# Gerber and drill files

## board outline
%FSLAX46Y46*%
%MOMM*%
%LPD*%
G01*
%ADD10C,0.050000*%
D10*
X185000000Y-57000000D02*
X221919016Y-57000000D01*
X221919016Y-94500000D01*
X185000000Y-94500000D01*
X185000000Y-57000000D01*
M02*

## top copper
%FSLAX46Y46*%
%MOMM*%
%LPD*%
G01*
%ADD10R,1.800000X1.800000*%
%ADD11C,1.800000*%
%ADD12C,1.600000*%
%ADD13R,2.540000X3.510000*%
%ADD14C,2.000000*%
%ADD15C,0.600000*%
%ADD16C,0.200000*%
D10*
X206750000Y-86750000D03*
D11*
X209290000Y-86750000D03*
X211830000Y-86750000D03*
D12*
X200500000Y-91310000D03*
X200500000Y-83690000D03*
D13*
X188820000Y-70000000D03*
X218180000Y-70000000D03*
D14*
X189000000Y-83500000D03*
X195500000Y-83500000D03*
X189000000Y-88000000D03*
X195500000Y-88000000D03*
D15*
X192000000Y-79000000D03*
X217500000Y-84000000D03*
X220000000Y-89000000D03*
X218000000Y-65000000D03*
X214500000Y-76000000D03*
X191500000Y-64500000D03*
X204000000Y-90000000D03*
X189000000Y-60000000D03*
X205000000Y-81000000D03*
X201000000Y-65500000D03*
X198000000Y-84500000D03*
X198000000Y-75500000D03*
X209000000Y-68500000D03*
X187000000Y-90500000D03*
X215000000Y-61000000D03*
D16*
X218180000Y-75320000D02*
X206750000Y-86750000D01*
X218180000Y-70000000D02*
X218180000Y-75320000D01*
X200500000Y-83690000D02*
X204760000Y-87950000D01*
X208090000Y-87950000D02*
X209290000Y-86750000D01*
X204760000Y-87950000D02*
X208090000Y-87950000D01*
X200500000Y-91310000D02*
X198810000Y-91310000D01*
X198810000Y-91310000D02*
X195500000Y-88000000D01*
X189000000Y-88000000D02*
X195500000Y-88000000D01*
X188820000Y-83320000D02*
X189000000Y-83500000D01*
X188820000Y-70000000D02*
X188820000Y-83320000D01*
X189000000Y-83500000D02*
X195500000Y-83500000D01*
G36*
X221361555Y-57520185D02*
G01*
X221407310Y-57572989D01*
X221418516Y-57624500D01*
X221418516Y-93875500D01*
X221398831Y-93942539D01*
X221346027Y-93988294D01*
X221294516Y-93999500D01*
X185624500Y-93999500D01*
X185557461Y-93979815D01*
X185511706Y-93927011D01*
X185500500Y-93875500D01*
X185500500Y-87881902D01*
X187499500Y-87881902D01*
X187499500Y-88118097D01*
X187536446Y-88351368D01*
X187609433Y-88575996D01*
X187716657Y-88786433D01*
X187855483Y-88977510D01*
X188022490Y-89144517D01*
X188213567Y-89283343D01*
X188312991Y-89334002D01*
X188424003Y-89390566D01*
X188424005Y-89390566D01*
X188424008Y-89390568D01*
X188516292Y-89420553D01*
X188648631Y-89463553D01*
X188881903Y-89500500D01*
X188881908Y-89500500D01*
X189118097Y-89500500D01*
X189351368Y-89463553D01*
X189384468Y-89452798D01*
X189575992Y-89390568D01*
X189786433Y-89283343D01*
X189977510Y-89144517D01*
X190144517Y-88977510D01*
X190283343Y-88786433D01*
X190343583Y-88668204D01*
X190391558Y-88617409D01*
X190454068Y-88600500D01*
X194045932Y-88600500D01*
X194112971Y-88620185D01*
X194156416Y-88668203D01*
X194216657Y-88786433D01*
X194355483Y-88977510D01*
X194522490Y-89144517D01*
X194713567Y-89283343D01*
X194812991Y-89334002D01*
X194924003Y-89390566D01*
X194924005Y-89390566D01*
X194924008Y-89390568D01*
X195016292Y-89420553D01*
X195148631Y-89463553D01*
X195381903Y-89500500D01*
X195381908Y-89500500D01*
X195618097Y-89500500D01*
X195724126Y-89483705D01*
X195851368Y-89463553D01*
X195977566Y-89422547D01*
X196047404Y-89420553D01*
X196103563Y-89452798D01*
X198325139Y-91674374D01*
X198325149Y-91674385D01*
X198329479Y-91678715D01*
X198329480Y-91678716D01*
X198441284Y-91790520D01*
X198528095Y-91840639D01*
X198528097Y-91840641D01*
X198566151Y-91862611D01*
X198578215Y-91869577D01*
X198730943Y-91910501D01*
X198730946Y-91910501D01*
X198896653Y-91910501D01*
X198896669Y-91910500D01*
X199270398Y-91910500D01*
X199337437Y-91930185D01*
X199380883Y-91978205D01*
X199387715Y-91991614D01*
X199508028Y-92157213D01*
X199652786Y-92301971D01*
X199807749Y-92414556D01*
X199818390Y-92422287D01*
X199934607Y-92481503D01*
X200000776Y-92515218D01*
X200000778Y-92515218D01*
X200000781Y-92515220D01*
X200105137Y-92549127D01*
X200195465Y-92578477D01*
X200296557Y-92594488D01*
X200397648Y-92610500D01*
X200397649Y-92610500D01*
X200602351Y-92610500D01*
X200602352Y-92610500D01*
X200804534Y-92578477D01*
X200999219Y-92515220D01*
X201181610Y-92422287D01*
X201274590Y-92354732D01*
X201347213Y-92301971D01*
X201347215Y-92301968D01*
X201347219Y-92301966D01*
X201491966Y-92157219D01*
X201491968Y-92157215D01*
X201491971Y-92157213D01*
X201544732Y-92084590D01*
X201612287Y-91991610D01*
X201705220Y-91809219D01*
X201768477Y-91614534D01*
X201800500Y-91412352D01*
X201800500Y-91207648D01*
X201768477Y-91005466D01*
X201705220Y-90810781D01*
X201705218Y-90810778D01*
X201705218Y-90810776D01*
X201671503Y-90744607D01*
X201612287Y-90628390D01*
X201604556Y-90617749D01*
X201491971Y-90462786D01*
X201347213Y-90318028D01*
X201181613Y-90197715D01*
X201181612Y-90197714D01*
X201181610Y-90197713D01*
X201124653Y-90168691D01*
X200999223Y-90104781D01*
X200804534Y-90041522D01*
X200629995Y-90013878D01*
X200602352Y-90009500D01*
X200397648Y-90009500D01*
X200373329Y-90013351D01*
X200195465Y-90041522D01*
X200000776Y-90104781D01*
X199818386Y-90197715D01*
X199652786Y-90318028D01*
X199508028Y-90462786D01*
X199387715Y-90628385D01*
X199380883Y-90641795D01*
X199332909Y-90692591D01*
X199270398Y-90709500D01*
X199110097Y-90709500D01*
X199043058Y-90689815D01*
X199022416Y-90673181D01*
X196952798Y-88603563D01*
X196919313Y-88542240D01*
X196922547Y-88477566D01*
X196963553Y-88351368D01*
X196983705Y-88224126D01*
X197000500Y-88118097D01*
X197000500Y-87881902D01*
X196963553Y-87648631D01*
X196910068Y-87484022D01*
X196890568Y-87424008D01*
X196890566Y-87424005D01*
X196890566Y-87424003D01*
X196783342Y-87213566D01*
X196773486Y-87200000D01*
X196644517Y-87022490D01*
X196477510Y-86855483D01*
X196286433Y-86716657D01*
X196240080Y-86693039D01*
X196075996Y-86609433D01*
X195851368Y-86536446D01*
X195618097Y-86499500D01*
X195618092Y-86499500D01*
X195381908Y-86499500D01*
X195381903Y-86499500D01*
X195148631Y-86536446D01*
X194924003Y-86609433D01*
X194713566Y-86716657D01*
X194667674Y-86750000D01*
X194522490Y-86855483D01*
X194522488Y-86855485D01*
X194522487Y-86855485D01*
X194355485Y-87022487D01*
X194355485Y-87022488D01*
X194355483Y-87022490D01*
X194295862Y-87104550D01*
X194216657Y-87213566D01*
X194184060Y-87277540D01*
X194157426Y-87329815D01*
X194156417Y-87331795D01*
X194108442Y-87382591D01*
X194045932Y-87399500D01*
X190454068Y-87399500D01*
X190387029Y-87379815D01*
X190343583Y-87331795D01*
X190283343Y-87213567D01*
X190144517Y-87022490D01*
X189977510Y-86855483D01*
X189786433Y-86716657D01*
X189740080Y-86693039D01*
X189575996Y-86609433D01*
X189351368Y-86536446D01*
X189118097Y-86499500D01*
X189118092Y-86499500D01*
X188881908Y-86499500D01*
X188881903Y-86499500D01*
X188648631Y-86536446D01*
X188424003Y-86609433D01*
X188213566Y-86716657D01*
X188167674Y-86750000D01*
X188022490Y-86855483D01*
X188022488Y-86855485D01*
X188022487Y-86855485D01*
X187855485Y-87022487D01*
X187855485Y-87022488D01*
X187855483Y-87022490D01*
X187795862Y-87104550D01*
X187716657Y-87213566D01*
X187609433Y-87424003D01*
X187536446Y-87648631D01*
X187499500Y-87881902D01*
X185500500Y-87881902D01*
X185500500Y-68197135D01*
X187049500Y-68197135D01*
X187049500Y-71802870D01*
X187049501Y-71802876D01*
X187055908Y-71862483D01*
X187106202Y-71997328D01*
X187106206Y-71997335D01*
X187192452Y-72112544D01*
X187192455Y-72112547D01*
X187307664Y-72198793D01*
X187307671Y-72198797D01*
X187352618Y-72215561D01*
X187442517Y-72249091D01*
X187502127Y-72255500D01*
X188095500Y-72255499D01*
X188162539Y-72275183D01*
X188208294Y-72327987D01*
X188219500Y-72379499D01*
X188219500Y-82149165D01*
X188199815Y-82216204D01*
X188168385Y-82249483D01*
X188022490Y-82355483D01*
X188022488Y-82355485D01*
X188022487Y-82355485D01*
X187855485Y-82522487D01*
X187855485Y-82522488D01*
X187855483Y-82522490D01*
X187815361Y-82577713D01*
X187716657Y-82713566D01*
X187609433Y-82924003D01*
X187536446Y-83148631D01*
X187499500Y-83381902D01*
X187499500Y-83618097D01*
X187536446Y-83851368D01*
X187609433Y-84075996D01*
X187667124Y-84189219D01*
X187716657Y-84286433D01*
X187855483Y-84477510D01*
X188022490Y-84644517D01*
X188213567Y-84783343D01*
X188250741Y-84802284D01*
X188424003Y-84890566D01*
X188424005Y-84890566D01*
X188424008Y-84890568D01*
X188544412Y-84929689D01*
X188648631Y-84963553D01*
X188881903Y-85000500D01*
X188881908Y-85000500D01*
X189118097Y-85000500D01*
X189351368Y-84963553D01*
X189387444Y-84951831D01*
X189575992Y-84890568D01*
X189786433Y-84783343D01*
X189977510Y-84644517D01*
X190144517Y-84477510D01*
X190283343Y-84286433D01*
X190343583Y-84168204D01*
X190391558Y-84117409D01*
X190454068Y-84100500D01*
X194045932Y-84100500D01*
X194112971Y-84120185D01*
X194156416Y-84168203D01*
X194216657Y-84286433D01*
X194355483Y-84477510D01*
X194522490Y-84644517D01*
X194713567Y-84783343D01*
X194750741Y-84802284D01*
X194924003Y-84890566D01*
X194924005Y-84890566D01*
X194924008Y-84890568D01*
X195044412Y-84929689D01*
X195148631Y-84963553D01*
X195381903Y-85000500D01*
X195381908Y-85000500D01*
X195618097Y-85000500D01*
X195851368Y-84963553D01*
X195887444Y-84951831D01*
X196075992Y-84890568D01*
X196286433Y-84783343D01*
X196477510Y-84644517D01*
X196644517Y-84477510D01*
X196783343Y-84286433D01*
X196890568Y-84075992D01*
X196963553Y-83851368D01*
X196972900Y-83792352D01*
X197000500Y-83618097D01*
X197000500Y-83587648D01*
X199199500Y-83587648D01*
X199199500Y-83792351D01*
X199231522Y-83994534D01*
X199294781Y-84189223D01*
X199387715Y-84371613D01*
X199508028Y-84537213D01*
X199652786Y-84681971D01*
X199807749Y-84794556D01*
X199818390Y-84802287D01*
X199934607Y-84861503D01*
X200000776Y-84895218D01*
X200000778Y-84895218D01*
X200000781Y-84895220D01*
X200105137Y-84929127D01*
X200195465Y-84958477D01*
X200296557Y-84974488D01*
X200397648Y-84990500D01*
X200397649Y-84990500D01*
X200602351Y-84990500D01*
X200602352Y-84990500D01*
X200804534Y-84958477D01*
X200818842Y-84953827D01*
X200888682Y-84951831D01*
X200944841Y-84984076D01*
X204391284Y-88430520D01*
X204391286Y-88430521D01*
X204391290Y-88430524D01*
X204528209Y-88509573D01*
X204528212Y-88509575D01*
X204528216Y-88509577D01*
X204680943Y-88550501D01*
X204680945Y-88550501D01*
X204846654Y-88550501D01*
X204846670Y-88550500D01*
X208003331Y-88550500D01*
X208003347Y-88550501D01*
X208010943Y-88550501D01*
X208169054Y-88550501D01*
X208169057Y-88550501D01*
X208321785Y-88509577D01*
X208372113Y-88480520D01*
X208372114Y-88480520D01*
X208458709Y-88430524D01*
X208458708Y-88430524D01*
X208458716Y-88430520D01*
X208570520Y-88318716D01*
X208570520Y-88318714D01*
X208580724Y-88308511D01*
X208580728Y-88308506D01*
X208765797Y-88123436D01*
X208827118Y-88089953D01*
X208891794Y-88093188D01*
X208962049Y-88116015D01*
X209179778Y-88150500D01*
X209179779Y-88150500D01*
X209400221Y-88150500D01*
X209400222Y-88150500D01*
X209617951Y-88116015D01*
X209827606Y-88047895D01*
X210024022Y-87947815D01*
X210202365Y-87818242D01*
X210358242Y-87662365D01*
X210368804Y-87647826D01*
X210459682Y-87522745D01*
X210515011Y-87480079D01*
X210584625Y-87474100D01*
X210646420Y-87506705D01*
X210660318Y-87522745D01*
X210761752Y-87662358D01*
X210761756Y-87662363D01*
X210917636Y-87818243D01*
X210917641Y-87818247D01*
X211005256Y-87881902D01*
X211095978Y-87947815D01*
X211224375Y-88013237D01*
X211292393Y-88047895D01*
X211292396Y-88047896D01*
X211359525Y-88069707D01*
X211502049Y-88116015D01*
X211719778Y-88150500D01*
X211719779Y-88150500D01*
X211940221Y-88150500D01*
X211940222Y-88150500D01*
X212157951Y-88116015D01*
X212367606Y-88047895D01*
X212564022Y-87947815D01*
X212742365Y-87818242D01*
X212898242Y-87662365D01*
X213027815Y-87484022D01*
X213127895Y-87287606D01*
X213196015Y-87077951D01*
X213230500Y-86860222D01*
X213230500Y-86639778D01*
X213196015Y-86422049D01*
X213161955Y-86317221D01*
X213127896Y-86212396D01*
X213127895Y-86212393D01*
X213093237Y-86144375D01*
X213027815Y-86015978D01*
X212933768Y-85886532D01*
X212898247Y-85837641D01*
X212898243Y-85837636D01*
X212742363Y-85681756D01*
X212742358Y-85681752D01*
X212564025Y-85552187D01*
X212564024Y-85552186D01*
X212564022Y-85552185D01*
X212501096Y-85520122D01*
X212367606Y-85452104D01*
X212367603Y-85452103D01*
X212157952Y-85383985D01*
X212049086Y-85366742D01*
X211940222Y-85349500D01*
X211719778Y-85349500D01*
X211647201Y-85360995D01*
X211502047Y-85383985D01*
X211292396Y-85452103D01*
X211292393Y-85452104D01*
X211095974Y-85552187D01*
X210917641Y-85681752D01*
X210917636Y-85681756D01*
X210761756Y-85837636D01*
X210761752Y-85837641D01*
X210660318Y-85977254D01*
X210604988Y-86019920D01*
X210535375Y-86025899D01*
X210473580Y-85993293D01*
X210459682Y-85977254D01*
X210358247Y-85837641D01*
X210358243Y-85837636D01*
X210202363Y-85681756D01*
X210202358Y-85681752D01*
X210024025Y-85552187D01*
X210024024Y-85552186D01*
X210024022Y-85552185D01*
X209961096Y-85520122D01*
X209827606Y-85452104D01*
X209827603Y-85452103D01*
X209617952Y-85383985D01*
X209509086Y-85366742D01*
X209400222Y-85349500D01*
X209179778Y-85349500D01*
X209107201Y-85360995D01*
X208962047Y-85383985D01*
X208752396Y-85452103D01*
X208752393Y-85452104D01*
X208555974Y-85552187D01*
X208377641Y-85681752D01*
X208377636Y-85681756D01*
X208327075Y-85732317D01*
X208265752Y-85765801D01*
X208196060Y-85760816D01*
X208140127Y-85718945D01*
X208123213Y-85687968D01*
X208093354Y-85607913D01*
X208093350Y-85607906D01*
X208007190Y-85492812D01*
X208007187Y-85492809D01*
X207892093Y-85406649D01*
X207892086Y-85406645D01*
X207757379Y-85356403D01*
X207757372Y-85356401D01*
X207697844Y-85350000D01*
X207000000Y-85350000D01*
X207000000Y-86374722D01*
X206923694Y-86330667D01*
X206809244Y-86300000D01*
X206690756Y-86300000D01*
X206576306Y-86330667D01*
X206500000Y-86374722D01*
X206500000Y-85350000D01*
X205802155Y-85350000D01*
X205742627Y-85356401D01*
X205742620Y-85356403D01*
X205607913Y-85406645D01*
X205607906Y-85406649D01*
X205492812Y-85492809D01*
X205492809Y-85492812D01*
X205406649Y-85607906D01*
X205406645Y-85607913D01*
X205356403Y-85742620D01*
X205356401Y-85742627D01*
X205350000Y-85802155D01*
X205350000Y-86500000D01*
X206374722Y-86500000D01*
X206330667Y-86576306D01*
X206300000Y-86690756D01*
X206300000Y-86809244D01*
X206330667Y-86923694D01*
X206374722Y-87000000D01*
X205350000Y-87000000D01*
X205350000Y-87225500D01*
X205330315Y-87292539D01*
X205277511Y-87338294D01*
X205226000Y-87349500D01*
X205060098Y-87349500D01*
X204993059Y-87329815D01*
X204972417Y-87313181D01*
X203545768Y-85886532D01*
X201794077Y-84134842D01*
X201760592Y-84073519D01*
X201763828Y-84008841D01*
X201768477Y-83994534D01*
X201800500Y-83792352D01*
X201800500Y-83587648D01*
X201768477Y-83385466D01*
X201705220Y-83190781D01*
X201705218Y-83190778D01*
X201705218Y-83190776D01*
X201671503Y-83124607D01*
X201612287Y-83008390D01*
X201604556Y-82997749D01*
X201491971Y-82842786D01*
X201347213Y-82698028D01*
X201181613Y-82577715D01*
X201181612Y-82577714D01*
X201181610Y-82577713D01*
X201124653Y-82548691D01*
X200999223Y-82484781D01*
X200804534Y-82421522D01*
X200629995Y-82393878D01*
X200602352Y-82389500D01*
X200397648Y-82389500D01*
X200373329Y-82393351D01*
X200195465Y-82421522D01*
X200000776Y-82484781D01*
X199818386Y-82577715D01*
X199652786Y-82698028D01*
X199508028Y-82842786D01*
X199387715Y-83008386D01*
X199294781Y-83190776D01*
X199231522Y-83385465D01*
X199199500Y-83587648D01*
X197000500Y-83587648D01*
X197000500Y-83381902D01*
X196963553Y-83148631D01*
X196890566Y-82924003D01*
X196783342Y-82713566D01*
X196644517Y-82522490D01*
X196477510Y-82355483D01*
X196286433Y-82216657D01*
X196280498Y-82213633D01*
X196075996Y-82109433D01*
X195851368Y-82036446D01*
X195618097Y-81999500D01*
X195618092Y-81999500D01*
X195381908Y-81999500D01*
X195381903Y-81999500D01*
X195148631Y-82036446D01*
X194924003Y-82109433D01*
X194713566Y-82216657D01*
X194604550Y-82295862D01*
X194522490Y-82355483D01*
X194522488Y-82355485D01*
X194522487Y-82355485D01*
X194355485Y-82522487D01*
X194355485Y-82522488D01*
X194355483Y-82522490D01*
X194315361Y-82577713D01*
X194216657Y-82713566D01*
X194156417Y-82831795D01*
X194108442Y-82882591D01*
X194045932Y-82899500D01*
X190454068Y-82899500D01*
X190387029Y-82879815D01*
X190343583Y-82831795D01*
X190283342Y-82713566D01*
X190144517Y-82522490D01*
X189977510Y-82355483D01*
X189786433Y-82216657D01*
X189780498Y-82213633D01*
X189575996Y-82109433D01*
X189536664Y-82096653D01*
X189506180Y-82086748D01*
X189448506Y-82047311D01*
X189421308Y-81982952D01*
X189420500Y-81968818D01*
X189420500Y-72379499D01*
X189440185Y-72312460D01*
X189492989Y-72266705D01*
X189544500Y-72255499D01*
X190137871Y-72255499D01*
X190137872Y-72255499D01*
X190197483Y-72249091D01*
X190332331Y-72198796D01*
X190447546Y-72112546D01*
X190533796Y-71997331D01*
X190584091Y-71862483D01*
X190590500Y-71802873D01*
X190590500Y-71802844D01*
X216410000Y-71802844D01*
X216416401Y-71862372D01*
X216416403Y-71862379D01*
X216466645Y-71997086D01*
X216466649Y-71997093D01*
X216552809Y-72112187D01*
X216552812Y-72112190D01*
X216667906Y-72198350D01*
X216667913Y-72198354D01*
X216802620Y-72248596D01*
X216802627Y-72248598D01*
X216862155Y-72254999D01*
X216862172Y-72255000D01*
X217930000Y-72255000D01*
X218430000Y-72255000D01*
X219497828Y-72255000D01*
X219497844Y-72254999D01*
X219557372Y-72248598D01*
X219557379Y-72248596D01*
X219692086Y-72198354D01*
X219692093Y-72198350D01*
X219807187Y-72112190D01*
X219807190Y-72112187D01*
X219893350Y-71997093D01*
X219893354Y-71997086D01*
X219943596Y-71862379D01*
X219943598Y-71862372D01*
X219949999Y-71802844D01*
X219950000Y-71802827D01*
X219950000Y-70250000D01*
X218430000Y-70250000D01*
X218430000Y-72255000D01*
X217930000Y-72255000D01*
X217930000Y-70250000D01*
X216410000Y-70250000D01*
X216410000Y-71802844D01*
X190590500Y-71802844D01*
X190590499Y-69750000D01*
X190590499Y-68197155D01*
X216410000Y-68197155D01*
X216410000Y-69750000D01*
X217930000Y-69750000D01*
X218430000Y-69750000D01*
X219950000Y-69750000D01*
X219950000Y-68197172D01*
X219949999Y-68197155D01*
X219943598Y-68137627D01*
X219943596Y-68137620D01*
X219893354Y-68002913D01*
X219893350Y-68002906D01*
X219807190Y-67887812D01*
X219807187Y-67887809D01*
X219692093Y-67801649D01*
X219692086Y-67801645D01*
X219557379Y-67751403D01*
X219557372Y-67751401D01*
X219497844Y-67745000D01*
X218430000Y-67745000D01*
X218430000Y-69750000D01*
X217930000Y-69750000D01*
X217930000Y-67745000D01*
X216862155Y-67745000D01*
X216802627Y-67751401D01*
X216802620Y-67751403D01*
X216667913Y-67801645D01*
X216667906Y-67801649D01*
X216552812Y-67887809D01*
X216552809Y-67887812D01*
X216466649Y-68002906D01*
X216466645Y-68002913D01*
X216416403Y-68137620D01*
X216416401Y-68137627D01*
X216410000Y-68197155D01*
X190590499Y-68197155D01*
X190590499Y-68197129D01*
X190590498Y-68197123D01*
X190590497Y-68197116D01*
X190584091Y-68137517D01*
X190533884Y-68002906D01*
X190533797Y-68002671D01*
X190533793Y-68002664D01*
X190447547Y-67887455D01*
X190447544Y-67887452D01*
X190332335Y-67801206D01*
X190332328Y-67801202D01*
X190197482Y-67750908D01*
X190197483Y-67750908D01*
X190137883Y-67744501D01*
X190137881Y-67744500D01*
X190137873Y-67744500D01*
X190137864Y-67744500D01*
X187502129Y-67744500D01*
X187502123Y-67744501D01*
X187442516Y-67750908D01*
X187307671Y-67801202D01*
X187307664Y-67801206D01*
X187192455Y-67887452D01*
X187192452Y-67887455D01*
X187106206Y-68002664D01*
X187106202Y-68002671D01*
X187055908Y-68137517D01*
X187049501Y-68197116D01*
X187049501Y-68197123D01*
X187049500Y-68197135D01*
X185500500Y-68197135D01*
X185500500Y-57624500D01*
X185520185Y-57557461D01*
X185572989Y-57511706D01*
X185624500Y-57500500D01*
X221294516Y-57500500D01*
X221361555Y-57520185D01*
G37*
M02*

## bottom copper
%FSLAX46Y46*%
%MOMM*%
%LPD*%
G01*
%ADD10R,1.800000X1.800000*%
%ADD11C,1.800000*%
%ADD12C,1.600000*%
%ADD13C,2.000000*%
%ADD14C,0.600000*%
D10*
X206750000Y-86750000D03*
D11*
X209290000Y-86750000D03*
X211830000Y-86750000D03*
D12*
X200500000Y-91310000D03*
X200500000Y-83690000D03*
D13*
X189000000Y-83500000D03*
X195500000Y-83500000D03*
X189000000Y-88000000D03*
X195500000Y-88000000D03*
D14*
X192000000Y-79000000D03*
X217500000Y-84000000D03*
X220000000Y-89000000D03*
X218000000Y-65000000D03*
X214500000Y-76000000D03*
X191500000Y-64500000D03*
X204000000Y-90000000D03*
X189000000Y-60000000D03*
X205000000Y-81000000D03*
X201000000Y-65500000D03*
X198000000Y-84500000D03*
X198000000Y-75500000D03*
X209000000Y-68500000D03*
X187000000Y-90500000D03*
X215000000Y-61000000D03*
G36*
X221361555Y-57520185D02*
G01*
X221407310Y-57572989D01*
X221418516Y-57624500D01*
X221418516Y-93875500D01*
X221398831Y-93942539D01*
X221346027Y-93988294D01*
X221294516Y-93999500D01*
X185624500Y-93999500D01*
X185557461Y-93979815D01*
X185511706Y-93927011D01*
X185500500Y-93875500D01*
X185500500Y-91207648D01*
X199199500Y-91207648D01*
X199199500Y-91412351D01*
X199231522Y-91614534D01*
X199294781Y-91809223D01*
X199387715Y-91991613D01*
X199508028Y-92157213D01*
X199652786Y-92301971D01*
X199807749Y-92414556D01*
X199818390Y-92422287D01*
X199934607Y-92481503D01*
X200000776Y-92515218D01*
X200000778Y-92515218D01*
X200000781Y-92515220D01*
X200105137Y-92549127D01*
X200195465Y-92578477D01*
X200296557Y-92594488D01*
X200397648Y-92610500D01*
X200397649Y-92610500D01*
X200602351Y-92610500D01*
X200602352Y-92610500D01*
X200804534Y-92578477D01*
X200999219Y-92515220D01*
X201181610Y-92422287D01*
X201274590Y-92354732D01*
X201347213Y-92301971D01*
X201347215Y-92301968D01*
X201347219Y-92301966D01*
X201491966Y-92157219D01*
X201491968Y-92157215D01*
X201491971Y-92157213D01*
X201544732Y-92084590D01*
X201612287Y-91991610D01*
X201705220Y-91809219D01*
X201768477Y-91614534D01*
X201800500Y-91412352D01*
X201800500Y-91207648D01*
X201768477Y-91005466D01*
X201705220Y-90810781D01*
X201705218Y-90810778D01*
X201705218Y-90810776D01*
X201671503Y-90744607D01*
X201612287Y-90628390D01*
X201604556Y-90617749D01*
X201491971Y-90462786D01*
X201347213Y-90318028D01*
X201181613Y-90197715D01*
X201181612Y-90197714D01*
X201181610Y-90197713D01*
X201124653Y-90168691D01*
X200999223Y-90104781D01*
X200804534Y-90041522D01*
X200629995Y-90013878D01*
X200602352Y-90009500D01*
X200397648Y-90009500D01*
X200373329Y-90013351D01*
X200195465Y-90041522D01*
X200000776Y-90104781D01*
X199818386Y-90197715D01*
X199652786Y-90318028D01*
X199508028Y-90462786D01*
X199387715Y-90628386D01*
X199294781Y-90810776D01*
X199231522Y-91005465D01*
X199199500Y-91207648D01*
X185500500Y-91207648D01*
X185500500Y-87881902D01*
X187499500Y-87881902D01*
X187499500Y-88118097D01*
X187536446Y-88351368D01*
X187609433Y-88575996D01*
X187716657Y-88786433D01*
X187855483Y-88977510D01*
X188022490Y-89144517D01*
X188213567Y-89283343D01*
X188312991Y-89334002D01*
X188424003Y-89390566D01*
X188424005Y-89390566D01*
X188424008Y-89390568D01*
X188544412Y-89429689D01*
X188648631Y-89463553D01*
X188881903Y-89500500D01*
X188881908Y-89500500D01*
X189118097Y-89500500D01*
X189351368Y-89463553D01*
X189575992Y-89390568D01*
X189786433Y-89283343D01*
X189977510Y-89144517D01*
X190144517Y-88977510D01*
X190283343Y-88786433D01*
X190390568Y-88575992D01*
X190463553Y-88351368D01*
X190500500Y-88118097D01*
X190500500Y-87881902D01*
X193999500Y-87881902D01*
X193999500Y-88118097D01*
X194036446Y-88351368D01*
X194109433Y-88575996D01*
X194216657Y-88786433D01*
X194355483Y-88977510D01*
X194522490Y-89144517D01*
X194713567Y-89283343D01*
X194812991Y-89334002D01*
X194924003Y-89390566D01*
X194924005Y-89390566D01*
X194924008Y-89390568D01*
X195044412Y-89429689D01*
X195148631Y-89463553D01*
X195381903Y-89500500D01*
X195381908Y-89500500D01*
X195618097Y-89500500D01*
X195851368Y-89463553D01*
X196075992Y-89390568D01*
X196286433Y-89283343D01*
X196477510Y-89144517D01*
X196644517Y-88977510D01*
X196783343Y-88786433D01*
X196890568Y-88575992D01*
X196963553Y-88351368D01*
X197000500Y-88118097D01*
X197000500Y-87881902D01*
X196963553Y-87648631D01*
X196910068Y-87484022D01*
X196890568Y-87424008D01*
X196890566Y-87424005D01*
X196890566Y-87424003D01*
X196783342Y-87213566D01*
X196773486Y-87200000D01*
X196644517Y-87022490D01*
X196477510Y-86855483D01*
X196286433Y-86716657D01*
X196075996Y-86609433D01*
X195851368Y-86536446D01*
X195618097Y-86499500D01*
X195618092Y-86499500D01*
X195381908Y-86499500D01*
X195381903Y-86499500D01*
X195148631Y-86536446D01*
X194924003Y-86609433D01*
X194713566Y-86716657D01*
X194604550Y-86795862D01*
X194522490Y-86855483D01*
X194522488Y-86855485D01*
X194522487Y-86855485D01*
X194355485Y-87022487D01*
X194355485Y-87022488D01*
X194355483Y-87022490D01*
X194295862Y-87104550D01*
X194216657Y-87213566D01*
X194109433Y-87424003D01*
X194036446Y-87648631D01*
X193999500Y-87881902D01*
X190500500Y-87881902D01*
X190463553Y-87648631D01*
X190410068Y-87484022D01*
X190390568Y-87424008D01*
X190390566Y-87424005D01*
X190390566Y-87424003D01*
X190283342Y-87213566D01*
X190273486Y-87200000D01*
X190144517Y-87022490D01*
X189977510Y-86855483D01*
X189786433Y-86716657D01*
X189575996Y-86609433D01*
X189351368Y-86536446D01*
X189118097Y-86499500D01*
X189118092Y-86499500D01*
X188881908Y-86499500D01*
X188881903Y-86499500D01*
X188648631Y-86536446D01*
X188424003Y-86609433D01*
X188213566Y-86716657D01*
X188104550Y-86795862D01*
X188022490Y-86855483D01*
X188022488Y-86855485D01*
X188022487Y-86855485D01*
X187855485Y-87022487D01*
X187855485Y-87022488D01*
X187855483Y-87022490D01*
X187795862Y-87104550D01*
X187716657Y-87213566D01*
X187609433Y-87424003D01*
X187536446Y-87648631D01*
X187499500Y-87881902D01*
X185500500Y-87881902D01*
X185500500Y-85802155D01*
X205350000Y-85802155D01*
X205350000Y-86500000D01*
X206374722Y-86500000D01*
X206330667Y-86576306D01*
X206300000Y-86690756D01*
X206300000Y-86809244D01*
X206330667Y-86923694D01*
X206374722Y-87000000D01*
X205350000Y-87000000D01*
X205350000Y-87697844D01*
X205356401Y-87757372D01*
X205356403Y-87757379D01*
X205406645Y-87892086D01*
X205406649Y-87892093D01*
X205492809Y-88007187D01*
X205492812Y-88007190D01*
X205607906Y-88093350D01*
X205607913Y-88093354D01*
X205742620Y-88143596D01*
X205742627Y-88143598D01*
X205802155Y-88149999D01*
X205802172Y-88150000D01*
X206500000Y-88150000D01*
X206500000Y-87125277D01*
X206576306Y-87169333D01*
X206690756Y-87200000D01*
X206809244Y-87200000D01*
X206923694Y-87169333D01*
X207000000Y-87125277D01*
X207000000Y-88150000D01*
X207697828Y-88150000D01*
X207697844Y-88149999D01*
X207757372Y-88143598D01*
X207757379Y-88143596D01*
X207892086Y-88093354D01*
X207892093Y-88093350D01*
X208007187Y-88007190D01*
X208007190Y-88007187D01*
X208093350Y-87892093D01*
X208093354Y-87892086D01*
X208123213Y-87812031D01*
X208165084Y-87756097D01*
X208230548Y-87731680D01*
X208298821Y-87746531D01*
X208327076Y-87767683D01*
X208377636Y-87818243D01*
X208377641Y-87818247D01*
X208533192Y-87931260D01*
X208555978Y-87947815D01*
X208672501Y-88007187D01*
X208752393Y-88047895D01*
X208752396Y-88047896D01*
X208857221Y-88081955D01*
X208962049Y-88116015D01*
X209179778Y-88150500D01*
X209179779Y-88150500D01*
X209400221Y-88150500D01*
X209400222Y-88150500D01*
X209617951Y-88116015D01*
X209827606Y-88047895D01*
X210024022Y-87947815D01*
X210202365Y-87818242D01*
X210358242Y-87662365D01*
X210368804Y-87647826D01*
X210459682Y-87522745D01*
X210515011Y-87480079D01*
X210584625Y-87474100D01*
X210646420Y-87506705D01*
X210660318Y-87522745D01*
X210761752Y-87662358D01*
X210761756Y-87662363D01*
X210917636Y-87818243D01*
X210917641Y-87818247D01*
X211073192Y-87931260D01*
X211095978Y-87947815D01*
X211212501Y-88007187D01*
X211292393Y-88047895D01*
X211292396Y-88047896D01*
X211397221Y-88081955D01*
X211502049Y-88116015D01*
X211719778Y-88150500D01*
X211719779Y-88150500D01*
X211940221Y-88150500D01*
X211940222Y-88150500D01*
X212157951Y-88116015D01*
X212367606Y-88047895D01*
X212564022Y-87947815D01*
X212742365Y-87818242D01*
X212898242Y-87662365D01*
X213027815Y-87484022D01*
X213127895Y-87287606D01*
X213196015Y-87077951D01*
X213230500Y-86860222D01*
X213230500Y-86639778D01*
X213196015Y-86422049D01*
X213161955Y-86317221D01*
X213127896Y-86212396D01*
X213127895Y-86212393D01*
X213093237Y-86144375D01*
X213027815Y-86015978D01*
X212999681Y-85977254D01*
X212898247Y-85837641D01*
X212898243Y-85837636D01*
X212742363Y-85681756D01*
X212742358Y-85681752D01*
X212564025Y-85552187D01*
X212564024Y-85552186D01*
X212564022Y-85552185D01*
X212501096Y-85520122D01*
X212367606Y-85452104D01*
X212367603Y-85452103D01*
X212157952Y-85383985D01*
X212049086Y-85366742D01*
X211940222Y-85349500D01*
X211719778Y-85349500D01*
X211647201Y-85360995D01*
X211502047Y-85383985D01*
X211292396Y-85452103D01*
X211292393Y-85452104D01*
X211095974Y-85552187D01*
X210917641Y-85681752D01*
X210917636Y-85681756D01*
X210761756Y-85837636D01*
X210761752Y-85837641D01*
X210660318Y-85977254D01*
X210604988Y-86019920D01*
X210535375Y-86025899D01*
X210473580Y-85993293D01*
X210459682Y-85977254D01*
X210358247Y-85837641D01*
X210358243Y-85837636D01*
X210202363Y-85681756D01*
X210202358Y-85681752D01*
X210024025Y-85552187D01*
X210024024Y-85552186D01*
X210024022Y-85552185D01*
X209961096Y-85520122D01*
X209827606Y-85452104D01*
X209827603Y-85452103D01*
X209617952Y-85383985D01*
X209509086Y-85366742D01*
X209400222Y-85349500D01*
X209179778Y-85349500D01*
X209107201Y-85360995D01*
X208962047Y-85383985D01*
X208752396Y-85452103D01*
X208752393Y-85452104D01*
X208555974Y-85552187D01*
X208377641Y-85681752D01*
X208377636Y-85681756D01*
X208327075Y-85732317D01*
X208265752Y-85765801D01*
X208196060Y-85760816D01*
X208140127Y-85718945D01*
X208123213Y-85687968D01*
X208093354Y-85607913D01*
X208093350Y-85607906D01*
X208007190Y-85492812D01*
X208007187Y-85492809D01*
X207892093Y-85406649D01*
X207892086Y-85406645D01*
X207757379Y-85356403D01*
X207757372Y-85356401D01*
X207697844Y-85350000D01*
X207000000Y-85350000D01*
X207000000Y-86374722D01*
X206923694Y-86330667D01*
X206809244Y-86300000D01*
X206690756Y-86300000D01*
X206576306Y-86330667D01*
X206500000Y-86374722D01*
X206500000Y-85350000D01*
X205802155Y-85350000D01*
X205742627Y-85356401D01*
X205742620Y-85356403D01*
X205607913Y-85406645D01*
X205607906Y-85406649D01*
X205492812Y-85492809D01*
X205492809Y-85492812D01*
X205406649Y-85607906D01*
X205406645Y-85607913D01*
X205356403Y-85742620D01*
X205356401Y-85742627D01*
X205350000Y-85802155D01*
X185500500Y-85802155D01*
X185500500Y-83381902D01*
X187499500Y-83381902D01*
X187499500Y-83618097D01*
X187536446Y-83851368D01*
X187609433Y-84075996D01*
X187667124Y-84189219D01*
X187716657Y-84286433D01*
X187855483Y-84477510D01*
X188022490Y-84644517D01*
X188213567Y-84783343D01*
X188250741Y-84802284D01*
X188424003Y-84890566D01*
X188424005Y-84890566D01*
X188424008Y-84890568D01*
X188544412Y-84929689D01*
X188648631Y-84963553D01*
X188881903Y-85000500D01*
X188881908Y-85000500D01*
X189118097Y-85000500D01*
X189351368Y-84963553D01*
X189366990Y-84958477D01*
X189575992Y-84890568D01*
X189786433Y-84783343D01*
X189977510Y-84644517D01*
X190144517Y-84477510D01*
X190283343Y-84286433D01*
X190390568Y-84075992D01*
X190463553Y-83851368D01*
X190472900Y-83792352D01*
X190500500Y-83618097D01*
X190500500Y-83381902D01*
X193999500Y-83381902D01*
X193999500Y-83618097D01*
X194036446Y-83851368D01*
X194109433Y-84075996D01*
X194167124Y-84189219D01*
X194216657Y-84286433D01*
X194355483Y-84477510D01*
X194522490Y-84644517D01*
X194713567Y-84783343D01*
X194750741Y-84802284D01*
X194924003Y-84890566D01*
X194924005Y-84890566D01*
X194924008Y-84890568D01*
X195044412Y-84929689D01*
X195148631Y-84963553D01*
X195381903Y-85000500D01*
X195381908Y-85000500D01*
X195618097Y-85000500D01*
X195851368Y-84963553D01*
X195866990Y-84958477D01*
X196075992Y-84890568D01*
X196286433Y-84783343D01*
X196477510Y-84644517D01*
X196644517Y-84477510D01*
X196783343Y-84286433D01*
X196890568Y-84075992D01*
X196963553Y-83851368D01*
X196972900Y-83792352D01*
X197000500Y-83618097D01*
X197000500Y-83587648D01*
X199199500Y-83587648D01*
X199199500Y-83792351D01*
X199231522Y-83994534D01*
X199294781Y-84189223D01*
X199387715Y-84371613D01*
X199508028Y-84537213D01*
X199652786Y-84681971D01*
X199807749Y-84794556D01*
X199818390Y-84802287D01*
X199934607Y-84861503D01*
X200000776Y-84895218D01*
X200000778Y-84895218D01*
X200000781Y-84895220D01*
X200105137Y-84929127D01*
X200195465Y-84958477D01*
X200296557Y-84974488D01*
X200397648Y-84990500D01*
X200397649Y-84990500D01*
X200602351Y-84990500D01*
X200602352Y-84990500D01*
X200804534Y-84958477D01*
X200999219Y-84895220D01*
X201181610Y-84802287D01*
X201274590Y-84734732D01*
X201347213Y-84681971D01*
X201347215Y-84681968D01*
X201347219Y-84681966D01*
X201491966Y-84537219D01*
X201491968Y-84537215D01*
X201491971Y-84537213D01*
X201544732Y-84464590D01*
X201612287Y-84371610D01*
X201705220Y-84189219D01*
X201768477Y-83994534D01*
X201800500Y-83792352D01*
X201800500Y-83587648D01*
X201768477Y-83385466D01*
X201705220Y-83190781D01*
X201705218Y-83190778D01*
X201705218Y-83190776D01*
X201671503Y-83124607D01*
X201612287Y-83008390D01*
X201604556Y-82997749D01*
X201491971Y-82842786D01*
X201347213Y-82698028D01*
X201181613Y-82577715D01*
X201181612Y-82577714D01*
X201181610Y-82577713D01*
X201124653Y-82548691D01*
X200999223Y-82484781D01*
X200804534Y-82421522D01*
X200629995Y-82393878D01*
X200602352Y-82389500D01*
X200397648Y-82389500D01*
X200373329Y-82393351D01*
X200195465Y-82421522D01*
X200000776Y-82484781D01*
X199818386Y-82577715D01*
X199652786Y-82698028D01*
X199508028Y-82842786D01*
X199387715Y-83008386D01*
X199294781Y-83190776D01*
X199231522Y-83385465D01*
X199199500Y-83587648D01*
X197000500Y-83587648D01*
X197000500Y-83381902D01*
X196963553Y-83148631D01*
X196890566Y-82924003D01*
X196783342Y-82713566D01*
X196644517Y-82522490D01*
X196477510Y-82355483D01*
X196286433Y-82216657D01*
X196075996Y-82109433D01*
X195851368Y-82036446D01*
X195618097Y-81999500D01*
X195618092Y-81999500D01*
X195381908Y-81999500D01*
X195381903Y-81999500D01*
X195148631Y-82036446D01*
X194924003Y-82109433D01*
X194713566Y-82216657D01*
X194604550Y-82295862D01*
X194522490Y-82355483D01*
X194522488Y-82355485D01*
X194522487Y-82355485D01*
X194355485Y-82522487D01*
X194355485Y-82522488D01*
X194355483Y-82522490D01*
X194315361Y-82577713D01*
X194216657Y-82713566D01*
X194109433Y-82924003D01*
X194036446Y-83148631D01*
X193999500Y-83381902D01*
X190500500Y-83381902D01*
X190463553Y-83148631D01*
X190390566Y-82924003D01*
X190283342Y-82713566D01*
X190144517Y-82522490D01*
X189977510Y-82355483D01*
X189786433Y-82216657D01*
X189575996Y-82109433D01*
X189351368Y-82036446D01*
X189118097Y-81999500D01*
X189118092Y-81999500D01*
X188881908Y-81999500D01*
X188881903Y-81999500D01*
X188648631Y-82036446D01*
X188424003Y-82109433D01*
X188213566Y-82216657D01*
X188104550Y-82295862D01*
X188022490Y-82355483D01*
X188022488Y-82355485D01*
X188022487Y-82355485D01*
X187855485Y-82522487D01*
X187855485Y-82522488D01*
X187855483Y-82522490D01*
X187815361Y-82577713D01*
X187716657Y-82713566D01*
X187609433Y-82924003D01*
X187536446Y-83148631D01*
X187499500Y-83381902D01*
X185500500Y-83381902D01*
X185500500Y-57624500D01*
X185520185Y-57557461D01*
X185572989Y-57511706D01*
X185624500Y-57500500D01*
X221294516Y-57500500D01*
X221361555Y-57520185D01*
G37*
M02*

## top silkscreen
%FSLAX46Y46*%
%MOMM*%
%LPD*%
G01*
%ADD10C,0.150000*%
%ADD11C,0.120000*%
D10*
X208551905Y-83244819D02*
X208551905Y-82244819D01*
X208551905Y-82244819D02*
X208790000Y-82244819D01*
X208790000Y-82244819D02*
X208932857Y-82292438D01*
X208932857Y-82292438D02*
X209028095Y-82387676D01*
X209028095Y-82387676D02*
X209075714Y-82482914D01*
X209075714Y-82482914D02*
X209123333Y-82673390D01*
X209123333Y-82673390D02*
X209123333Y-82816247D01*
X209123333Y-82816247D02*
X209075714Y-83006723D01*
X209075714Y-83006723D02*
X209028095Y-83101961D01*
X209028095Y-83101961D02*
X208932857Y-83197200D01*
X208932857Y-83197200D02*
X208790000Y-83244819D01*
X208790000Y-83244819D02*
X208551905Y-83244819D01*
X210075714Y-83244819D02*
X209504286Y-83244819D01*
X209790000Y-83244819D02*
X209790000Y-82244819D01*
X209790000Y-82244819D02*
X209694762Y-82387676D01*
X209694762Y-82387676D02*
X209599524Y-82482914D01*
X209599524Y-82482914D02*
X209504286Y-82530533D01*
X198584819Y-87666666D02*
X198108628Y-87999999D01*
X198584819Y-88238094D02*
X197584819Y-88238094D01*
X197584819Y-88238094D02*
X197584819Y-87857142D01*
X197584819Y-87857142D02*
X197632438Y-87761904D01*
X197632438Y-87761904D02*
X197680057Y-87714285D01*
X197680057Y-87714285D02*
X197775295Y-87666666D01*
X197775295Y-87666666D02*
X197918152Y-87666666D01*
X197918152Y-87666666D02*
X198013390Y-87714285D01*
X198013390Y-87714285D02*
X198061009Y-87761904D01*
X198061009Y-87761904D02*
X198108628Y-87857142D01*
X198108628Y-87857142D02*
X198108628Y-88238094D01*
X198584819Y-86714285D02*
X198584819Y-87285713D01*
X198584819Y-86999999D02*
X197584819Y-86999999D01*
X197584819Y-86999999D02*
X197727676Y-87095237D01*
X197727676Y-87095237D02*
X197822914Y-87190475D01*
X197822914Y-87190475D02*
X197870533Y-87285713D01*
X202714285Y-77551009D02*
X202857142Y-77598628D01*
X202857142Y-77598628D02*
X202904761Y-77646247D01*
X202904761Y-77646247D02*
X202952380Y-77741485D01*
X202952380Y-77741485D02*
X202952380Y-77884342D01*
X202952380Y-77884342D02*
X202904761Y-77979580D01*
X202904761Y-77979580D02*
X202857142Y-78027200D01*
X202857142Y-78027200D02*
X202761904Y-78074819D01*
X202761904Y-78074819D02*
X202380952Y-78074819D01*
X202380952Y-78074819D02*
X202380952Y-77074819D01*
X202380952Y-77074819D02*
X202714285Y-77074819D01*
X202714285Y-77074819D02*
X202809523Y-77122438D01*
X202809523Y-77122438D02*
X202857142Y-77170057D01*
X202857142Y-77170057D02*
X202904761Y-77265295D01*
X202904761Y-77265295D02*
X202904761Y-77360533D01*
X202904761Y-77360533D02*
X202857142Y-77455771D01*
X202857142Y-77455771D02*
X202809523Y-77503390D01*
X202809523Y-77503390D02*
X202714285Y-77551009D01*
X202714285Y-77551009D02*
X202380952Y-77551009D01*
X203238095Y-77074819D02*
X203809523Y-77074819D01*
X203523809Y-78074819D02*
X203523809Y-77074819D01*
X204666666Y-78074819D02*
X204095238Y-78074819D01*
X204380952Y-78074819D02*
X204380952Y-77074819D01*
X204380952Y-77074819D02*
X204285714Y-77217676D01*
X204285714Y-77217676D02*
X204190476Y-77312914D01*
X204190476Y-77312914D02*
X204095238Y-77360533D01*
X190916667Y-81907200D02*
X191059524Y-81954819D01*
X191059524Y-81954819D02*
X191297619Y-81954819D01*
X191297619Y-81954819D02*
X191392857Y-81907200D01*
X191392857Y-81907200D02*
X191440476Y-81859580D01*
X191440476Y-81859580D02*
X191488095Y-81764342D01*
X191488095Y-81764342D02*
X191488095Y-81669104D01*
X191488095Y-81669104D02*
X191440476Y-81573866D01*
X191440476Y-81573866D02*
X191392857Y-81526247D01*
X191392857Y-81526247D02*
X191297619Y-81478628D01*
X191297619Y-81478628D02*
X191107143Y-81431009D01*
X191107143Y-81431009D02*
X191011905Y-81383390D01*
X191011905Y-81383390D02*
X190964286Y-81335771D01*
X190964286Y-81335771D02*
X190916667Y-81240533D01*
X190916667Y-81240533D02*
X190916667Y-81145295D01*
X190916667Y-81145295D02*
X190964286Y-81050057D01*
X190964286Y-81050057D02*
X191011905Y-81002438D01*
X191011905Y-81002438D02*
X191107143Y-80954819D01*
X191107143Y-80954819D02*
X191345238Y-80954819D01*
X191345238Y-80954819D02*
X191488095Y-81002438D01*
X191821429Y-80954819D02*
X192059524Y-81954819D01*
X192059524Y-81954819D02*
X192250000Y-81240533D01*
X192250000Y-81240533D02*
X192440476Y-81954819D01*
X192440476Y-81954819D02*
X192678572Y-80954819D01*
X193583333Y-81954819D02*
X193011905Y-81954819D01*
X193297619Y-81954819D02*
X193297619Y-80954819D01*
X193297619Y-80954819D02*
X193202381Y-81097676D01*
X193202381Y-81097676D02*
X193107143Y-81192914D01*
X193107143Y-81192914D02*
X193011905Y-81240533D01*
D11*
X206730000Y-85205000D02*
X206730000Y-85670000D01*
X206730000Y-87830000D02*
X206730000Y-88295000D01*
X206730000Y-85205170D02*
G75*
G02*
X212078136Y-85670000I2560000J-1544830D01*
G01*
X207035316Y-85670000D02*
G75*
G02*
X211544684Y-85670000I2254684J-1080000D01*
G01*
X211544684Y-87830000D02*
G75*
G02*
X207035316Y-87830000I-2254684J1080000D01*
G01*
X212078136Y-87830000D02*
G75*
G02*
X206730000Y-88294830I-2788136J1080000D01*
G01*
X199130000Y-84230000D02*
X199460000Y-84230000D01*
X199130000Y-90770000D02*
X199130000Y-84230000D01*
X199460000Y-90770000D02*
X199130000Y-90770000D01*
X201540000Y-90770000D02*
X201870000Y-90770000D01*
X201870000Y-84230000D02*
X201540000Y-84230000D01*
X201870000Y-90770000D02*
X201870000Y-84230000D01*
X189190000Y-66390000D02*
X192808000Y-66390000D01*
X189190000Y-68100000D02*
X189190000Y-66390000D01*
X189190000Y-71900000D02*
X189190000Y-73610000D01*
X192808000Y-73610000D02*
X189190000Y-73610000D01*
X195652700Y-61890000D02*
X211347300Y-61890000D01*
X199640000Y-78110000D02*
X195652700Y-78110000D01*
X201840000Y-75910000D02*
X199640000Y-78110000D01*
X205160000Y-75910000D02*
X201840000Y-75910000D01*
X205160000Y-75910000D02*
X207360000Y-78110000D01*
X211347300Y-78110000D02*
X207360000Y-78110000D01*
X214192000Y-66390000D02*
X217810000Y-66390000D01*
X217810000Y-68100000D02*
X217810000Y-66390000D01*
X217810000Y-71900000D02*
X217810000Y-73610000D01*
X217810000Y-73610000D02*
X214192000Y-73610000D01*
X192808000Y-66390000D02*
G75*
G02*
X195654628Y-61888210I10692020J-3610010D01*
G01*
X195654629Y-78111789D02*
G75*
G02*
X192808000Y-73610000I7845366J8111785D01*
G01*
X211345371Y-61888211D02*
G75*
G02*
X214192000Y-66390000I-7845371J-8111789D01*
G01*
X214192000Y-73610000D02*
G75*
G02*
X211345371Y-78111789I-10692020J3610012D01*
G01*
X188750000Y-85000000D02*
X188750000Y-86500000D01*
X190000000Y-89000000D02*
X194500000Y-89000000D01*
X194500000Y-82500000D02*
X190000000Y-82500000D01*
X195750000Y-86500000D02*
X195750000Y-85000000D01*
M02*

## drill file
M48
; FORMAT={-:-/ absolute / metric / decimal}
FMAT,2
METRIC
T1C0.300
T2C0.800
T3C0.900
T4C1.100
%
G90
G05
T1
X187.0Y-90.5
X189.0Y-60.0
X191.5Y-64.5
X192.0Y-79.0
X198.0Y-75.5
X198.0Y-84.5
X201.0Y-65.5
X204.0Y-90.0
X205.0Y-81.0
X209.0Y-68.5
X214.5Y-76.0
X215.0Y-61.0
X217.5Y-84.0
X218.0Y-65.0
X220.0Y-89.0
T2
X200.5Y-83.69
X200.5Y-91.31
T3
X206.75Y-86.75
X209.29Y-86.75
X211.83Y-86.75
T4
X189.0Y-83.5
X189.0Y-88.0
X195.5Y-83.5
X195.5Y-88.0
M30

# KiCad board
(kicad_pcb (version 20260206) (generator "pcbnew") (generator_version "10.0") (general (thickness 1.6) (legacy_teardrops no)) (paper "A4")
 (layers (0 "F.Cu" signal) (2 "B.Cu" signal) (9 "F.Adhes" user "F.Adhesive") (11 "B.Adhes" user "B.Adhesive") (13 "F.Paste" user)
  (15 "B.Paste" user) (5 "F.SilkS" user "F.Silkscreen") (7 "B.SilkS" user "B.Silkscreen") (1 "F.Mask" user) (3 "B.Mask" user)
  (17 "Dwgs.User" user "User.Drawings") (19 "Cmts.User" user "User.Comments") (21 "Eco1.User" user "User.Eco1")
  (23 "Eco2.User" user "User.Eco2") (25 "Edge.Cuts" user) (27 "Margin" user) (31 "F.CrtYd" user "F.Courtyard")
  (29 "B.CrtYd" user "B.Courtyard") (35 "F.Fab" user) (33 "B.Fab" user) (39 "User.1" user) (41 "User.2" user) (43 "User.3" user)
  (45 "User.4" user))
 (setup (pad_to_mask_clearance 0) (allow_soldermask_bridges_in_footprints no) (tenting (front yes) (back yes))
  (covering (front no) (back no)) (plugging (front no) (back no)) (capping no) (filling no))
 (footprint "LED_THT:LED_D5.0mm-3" (layer "F.Cu") (at 206.75 86.75)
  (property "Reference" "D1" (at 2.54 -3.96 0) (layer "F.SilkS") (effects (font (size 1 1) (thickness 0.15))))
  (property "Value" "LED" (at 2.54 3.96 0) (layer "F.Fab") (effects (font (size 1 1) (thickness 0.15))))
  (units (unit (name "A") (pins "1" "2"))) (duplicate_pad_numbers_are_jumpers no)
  (fp_line (start -0.02 -1.545) (end -0.02 -1.08) (stroke (width 0.12) (type solid)) (layer "F.SilkS"))
  (fp_line (start -0.02 1.08) (end -0.02 1.545) (stroke (width 0.12) (type solid)) (layer "F.SilkS"))
  (fp_arc (start -0.02 -1.54483) (mid 2.798898 -2.97877) (end 5.328136 -1.08) (stroke (width 0.12) (type solid)) (layer "F.SilkS"))
  (fp_arc (start 0.285316 -1.08) (mid 2.54 -2.5) (end 4.794684 -1.08) (stroke (width 0.12) (type solid)) (layer "F.SilkS"))
  (fp_arc (start 4.794684 1.08) (mid 2.54 2.5) (end 0.285316 1.08) (stroke (width 0.12) (type solid)) (layer "F.SilkS"))
  (fp_arc (start 5.328136 1.08) (mid 2.798898 2.97877) (end -0.02 1.54483) (stroke (width 0.12) (type solid)) (layer "F.SilkS"))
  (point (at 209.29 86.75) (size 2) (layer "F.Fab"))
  (pad "1" thru_hole rect (at 0 0) (size 1.8 1.8) (drill 0.9) (layers "*.Cu" "*.Mask") (remove_unused_layers no) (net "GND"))
  (pad "2" thru_hole circle (at 2.54 0) (size 1.8 1.8) (drill 0.9) (layers "*.Cu" "*.Mask") (remove_unused_layers no) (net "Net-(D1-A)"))
  (pad "3" thru_hole circle (at 5.08 0) (size 1.8 1.8) (drill 0.9) (layers "*.Cu" "*.Mask") (remove_unused_layers no)))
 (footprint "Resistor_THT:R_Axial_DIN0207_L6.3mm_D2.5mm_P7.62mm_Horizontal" (layer "F.Cu") (at 200.5 91.31 90)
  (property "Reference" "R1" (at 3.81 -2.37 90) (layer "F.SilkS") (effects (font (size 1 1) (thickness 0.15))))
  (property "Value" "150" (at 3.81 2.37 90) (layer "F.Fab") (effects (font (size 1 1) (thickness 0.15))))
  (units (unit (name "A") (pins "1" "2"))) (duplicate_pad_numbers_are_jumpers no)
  (fp_line (start 7.08 -1.37) (end 7.08 -1.04) (stroke (width 0.12) (type solid)) (layer "F.SilkS"))
  (fp_line (start 0.54 -1.37) (end 7.08 -1.37) (stroke (width 0.12) (type solid)) (layer "F.SilkS"))
  (fp_line (start 0.54 -1.04) (end 0.54 -1.37) (stroke (width 0.12) (type solid)) (layer "F.SilkS"))
  (fp_line (start 0.54 1.04) (end 0.54 1.37) (stroke (width 0.12) (type solid)) (layer "F.SilkS"))
  (fp_line (start 7.08 1.37) (end 7.08 1.04) (stroke (width 0.12) (type solid)) (layer "F.SilkS"))
  (fp_line (start 0.54 1.37) (end 7.08 1.37) (stroke (width 0.12) (type solid)) (layer "F.SilkS"))
  (pad "1" thru_hole circle (at 0 0 90) (size 1.6 1.6) (drill 0.8) (layers "*.Cu" "*.Mask") (remove_unused_layers no) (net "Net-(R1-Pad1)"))
  (pad "2" thru_hole circle (at 7.62 0 90) (size 1.6 1.6) (drill 0.8) (layers "*.Cu" "*.Mask") (remove_unused_layers no) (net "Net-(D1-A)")))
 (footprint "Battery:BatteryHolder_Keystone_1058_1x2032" (layer "F.Cu") (at 203.5 70)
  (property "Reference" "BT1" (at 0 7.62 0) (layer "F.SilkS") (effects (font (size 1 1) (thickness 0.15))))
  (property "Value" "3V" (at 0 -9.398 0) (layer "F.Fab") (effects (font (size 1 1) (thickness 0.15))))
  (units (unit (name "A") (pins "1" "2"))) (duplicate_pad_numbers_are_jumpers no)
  (fp_line (start -14.31 -3.61) (end -10.692 -3.61) (stroke (width 0.12) (type solid)) (layer "F.SilkS"))
  (fp_line (start -14.31 -1.9) (end -14.31 -3.61) (stroke (width 0.12) (type solid)) (layer "F.SilkS"))
  (fp_line (start -14.31 1.9) (end -14.31 3.61) (stroke (width 0.12) (type solid)) (layer "F.SilkS"))
  (fp_line (start -10.692 3.61) (end -14.31 3.61) (stroke (width 0.12) (type solid)) (layer "F.SilkS"))
  (fp_line (start -7.8473 -8.11) (end 7.8473 -8.11) (stroke (width 0.12) (type solid)) (layer "F.SilkS"))
  (fp_line (start -3.86 8.11) (end -7.8473 8.11) (stroke (width 0.12) (type solid)) (layer "F.SilkS"))
  (fp_line (start -1.66 5.91) (end -3.86 8.11) (stroke (width 0.12) (type solid)) (layer "F.SilkS"))
  (fp_line (start 1.66 5.91) (end -1.66 5.91) (stroke (width 0.12) (type solid)) (layer "F.SilkS"))
  (fp_line (start 1.66 5.91) (end 3.86 8.11) (stroke (width 0.12) (type solid)) (layer "F.SilkS"))
  (fp_line (start 7.8473 8.11) (end 3.86 8.11) (stroke (width 0.12) (type solid)) (layer "F.SilkS"))
  (fp_line (start 10.692 -3.61) (end 14.31 -3.61) (stroke (width 0.12) (type solid)) (layer "F.SilkS"))
  (fp_line (start 14.31 -1.9) (end 14.31 -3.61) (stroke (width 0.12) (type solid)) (layer "F.SilkS"))
  (fp_line (start 14.31 1.9) (end 14.31 3.61) (stroke (width 0.12) (type solid)) (layer "F.SilkS"))
  (fp_line (start 14.31 3.61) (end 10.692 3.61) (stroke (width 0.12) (type solid)) (layer "F.SilkS"))
  (fp_arc (start -10.692 -3.61) (mid -9.538084 -6.031244) (end -7.845371 -8.111789) (stroke (width 0.12) (type solid)) (layer "F.SilkS"))
  (fp_arc (start -7.845371 8.111789) (mid -9.538085 6.031244) (end -10.692 3.61) (stroke (width 0.12) (type solid)) (layer "F.SilkS"))
  (fp_arc (start 7.845371 -8.111789) (mid 9.538085 -6.031244) (end 10.692 -3.61) (stroke (width 0.12) (type solid)) (layer "F.SilkS"))
  (fp_arc (start 10.692 3.61) (mid 9.538084 6.031244) (end 7.845371 8.111789) (stroke (width 0.12) (type solid)) (layer "F.SilkS"))
  (pad "1" smd rect (at -14.68 0) (size 2.54 3.51) (layers "F.Cu" "F.Mask" "F.Paste") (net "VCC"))
  (pad "2" smd rect (at 14.68 0) (size 2.54 3.51) (layers "F.Cu" "F.Mask" "F.Paste") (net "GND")))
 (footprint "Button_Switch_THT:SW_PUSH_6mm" (layer "F.Cu") (at 189 83.5)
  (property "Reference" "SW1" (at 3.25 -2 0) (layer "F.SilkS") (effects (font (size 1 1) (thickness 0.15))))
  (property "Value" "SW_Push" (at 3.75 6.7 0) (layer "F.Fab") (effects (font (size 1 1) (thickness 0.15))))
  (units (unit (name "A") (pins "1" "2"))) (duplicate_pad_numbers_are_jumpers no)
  (fp_line (start -0.25 1.5) (end -0.25 3) (stroke (width 0.12) (type solid)) (layer "F.SilkS"))
  (fp_line (start 1 5.5) (end 5.5 5.5) (stroke (width 0.12) (type solid)) (layer "F.SilkS"))
  (fp_line (start 5.5 -1) (end 1 -1) (stroke (width 0.12) (type solid)) (layer "F.SilkS"))
  (fp_line (start 6.75 3) (end 6.75 1.5) (stroke (width 0.12) (type solid)) (layer "F.SilkS"))
  (pad "1" thru_hole circle (at 0 0 90) (size 2 2) (drill 1.1) (layers "*.Cu" "*.Mask") (remove_unused_layers no) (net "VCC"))
  (pad "1" thru_hole circle (at 6.5 0 90) (size 2 2) (drill 1.1) (layers "*.Cu" "*.Mask") (remove_unused_layers no) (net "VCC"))
  (pad "2" thru_hole circle (at 0 4.5 90) (size 2 2) (drill 1.1) (layers "*.Cu" "*.Mask") (remove_unused_layers no) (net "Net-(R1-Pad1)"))
  (pad "2" thru_hole circle (at 6.5 4.5 90) (size 2 2) (drill 1.1) (layers "*.Cu" "*.Mask") (remove_unused_layers no) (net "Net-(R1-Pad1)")))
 (gr_rect (start 185 57) (end 221.919016 94.5) (stroke (width 0.05) (type default)) (fill no) (layer "Edge.Cuts"))
 (segment (start 218.18 75.32) (end 206.75 86.75) (width 0.2) (layer "F.Cu") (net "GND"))
 (segment (start 218.18 70) (end 218.18 75.32) (width 0.2) (layer "F.Cu") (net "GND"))
 (via (at 192 79) (size 0.6) (drill 0.3) (layers "F.Cu" "B.Cu") (free yes) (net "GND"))
 (via (at 217.5 84) (size 0.6) (drill 0.3) (layers "F.Cu" "B.Cu") (free yes) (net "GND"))
 (via (at 220 89) (size 0.6) (drill 0.3) (layers "F.Cu" "B.Cu") (free yes) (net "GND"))
 (via (at 218 65) (size 0.6) (drill 0.3) (layers "F.Cu" "B.Cu") (free yes) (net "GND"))
 (via (at 214.5 76) (size 0.6) (drill 0.3) (layers "F.Cu" "B.Cu") (free yes) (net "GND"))
 (via (at 191.5 64.5) (size 0.6) (drill 0.3) (layers "F.Cu" "B.Cu") (free yes) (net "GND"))
 (via (at 204 90) (size 0.6) (drill 0.3) (layers "F.Cu" "B.Cu") (free yes) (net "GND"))
 (via (at 189 60) (size 0.6) (drill 0.3) (layers "F.Cu" "B.Cu") (free yes) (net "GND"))
 (via (at 205 81) (size 0.6) (drill 0.3) (layers "F.Cu" "B.Cu") (free yes) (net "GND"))
 (via (at 201 65.5) (size 0.6) (drill 0.3) (layers "F.Cu" "B.Cu") (free yes) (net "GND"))
 (via (at 198 84.5) (size 0.6) (drill 0.3) (layers "F.Cu" "B.Cu") (free yes) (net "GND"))
 (via (at 198 75.5) (size 0.6) (drill 0.3) (layers "F.Cu" "B.Cu") (free yes) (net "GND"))
 (via (at 209 68.5) (size 0.6) (drill 0.3) (layers "F.Cu" "B.Cu") (free yes) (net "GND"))
 (via (at 187 90.5) (size 0.6) (drill 0.3) (layers "F.Cu" "B.Cu") (free yes) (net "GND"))
 (via (at 215 61) (size 0.6) (drill 0.3) (layers "F.Cu" "B.Cu") (free yes) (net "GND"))
 (segment (start 200.5 83.69) (end 204.76 87.95) (width 0.2) (layer "F.Cu") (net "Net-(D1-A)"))
 (segment (start 208.09 87.95) (end 209.29 86.75) (width 0.2) (layer "F.Cu") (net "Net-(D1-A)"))
 (segment (start 204.76 87.95) (end 208.09 87.95) (width 0.2) (layer "F.Cu") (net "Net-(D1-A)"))
 (segment (start 200.5 91.31) (end 198.81 91.31) (width 0.2) (layer "F.Cu") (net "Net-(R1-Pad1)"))
 (segment (start 198.81 91.31) (end 195.5 88) (width 0.2) (layer "F.Cu") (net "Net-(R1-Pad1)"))
 (segment (start 189 88) (end 195.5 88) (width 0.2) (layer "F.Cu") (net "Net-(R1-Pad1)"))
 (segment (start 188.82 83.32) (end 189 83.5) (width 0.2) (layer "F.Cu") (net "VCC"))
 (segment (start 188.82 70) (end 188.82 83.32) (width 0.2) (layer "F.Cu") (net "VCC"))
 (segment (start 189 83.5) (end 195.5 83.5) (width 0.2) (layer "F.Cu") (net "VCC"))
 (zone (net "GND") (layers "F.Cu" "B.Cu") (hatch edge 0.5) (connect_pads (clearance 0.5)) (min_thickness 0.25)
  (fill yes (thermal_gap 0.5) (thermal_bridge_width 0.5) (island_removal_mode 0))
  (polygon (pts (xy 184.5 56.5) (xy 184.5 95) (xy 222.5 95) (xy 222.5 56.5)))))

